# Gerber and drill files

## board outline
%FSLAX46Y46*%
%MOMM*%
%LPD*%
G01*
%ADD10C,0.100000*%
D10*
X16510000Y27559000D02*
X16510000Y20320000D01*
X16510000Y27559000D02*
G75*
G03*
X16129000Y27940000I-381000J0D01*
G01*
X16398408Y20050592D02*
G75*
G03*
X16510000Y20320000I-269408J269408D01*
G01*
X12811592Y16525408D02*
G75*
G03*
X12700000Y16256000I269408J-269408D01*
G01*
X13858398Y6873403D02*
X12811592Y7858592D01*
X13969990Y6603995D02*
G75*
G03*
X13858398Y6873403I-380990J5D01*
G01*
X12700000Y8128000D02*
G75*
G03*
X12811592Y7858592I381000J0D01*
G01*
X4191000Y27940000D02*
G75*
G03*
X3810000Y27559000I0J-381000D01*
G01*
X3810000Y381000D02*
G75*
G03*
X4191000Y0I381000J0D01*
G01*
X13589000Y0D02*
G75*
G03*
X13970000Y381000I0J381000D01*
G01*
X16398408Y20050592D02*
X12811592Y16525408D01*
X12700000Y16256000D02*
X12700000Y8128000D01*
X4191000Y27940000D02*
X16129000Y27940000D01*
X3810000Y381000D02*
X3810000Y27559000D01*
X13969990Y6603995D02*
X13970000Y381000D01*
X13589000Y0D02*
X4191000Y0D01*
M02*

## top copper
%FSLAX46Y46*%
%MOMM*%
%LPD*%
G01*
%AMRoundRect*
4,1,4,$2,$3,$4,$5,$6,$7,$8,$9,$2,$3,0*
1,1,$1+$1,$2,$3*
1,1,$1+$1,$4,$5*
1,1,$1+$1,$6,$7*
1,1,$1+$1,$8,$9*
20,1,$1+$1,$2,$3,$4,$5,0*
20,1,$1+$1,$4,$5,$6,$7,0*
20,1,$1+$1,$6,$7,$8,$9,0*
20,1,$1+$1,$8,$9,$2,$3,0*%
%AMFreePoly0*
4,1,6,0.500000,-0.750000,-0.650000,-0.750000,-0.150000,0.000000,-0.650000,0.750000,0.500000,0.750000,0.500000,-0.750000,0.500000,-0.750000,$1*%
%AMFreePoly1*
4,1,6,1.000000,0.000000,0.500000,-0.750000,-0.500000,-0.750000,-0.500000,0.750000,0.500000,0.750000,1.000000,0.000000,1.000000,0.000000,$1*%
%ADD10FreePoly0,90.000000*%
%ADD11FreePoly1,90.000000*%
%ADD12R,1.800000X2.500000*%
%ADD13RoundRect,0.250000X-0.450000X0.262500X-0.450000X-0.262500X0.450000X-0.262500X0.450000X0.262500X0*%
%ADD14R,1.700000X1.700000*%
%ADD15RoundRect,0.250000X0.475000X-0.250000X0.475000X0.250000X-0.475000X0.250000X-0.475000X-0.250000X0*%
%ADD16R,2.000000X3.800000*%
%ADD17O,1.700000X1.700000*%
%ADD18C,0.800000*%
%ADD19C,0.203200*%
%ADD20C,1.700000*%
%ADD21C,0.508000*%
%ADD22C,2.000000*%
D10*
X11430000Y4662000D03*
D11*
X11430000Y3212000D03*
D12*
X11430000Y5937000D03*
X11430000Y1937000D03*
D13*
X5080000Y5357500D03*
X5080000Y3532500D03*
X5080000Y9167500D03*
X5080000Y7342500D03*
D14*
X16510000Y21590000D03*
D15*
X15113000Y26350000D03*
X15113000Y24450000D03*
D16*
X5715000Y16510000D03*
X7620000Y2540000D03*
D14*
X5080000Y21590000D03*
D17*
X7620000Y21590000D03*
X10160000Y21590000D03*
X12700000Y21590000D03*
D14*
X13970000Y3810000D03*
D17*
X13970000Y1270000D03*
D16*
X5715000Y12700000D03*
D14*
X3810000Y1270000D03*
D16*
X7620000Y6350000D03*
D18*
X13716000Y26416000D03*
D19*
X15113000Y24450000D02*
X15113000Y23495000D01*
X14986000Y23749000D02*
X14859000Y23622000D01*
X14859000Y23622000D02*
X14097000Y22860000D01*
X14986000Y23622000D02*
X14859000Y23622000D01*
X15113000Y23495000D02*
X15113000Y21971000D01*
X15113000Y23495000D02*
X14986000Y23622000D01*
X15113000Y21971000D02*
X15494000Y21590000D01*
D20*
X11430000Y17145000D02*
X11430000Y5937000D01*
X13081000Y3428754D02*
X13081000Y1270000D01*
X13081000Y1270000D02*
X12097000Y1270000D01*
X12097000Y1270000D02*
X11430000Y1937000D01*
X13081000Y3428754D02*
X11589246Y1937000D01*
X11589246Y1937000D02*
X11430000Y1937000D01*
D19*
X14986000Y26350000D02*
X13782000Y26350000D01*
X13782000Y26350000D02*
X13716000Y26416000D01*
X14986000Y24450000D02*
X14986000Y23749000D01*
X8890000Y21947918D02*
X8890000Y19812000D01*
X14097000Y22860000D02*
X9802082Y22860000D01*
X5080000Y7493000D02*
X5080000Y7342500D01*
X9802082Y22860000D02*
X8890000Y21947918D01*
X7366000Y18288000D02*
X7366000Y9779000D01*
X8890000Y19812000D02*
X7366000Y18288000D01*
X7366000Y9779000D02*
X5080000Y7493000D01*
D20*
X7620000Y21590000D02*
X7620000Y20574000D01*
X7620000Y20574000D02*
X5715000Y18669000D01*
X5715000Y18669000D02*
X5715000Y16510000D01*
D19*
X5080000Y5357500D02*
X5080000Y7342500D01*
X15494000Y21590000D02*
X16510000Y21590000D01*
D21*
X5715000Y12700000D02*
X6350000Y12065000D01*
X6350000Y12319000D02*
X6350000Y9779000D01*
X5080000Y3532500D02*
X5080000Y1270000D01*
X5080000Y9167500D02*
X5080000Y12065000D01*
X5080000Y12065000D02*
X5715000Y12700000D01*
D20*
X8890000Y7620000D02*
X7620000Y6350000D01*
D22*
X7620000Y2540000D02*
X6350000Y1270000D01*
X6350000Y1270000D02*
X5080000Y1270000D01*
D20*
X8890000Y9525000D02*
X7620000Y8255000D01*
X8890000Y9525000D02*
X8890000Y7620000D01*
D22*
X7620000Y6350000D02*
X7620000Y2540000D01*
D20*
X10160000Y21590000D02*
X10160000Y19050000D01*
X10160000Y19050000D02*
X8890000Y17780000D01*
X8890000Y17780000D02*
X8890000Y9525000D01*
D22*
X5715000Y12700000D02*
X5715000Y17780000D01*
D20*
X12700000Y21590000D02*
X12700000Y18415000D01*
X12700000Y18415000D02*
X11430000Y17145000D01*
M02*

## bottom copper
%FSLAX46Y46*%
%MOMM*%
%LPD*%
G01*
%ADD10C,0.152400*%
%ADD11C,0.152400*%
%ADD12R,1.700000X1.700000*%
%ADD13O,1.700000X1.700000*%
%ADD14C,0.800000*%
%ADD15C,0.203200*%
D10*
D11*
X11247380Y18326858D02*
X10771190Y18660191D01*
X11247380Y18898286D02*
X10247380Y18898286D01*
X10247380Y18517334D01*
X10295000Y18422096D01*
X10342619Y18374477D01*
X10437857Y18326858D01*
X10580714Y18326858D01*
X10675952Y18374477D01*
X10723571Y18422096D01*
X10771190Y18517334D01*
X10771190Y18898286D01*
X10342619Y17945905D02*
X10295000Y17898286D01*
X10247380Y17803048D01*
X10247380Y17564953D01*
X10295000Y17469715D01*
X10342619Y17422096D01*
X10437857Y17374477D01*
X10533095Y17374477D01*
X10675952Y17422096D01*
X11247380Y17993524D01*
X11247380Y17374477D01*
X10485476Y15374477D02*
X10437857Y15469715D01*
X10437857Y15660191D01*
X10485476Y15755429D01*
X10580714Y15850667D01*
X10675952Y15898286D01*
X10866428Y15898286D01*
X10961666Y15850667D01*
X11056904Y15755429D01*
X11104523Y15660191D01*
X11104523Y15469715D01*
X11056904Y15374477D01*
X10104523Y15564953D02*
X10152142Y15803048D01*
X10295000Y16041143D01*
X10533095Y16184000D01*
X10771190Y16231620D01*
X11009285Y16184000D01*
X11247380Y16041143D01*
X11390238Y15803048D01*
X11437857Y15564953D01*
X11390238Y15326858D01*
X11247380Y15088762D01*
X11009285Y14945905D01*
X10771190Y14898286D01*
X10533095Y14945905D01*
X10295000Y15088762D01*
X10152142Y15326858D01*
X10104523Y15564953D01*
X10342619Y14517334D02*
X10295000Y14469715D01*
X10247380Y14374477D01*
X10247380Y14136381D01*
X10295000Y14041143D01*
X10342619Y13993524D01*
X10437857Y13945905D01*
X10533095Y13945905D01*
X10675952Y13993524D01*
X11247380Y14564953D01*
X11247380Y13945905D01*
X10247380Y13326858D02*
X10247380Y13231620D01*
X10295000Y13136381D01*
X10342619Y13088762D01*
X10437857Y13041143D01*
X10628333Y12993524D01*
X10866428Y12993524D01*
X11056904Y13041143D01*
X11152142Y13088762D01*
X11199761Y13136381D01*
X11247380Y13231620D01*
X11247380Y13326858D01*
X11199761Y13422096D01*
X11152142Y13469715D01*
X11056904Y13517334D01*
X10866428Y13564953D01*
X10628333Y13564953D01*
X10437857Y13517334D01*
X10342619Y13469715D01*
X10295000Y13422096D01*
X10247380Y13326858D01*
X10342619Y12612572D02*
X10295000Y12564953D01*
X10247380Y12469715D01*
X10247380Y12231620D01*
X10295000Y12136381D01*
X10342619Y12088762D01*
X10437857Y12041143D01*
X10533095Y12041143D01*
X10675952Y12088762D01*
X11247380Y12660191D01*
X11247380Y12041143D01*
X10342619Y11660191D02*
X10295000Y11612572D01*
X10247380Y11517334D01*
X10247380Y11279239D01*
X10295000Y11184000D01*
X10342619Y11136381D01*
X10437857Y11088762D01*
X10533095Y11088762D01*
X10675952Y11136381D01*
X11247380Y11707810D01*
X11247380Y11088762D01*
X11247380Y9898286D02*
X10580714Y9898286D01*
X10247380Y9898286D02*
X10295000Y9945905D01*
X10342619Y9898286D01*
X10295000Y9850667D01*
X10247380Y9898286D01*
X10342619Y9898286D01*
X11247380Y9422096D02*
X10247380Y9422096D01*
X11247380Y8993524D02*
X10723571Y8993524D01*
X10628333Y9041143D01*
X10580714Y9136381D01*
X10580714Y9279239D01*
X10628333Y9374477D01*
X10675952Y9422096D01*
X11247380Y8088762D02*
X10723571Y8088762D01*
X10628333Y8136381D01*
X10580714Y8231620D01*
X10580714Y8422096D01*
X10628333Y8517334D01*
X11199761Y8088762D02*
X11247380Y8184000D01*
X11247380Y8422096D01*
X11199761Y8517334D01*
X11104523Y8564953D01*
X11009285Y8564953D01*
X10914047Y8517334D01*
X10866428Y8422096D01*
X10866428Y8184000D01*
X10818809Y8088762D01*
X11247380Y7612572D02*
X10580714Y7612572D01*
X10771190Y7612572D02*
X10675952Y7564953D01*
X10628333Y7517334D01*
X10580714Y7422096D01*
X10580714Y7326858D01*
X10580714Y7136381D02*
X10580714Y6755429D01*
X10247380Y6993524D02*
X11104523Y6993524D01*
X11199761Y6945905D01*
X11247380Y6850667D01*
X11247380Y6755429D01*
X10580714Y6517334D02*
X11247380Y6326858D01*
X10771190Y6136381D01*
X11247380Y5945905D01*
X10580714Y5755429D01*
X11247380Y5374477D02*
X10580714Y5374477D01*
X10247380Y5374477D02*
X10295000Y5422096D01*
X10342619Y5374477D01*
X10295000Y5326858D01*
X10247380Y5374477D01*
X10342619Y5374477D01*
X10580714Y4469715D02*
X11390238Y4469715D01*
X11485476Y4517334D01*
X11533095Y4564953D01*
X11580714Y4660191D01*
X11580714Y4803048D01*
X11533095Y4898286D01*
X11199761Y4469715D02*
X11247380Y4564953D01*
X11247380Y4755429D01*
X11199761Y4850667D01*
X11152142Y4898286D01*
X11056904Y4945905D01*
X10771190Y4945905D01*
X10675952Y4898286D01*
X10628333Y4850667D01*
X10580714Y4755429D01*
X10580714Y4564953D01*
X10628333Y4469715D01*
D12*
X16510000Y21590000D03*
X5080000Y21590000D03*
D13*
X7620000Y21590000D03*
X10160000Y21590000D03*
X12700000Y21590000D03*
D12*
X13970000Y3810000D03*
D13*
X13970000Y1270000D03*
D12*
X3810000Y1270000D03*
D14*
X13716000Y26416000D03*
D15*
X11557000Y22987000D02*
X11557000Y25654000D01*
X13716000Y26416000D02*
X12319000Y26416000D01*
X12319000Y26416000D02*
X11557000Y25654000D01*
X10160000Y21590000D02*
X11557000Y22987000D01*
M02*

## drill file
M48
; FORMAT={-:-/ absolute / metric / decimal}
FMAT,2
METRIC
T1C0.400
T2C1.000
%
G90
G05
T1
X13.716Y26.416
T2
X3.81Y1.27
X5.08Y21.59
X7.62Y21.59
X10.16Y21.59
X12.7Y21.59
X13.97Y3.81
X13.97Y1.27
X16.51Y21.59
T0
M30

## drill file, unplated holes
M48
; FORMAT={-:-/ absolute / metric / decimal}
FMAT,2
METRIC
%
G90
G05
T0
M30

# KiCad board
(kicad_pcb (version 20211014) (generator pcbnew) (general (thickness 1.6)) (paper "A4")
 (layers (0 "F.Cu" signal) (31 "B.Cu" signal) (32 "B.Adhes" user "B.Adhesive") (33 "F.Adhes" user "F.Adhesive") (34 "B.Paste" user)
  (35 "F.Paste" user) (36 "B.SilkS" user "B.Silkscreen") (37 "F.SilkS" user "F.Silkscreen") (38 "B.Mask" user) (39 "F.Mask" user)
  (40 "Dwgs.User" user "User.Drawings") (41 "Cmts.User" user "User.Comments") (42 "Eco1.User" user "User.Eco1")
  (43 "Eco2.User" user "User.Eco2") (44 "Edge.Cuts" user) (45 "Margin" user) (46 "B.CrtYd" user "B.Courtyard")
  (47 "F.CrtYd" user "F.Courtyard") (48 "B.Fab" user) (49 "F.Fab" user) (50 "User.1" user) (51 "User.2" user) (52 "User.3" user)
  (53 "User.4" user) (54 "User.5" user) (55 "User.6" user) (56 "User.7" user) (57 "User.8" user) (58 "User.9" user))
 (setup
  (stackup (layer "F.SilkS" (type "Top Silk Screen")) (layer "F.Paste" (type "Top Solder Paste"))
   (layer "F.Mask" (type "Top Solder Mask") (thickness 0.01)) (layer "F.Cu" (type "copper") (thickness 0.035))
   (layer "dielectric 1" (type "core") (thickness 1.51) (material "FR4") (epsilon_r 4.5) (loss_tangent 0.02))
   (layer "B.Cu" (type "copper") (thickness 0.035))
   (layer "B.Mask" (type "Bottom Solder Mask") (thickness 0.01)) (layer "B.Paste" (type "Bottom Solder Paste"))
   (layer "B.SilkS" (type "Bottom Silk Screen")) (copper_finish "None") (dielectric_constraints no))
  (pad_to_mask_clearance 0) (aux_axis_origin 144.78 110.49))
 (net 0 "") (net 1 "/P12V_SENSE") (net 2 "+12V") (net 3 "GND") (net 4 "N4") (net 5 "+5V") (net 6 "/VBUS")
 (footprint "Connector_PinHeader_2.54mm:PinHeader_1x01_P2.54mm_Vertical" (layer "F.Cu") (at 161.29 88.9 90)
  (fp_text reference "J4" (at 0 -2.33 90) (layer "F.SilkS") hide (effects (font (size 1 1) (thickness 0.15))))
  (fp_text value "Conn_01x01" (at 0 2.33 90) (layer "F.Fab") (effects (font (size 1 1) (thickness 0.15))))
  (pad "1" thru_hole rect (at 0 0 90) (size 1.7 1.7) (drill 1) (layers *.Cu *.Mask) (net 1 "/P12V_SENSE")))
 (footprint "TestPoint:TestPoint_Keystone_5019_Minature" (layer "F.Cu") (at 150.495 93.98 90)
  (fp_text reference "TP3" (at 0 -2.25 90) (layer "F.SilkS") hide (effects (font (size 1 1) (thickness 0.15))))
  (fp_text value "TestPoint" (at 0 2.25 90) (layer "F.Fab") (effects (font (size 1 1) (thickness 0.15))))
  (pad "1" smd rect (at 0 0 90) (size 3.8 2) (layers "F.Cu" "F.Paste" "F.Mask") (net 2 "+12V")))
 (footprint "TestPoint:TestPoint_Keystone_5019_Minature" (layer "F.Cu") (at 152.4 107.95 90)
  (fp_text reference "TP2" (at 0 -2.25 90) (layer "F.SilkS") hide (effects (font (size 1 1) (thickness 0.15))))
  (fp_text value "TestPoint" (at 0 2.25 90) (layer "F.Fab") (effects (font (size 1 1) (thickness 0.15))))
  (pad "1" smd rect (at 0 0 90) (size 3.8 2) (layers "F.Cu" "F.Paste" "F.Mask") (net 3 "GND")))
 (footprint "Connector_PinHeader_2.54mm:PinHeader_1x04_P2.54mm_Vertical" (layer "F.Cu") (at 149.86 88.9 90)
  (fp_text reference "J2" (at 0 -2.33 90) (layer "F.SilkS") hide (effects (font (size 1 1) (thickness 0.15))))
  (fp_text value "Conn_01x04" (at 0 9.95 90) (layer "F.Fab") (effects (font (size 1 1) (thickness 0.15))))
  (pad "1" thru_hole rect (at 0 0 90) (size 1.7 1.7) (drill 1) (layers *.Cu *.Mask) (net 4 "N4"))
  (pad "2" thru_hole oval (at 0 2.54 90) (size 1.7 1.7) (drill 1) (layers *.Cu *.Mask) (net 2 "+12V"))
  (pad "3" thru_hole oval (at 0 5.08 90) (size 1.7 1.7) (drill 1) (layers *.Cu *.Mask) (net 3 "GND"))
  (pad "4" thru_hole oval (at 0 7.62 90) (size 1.7 1.7) (drill 1) (layers *.Cu *.Mask) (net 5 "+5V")))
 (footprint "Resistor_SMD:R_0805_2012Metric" (layer "F.Cu") (at 149.86 102.235 -90)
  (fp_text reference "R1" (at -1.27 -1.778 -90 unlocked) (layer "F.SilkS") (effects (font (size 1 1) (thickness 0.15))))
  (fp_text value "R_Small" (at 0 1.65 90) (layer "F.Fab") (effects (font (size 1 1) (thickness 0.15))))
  (pad "1" smd roundrect (at -0.9125 0 270) (size 1.025 1.4) (layers "F.Cu" "F.Paste" "F.Mask") (roundrect_rratio 0.243902439)
   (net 2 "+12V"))
  (pad "2" smd roundrect (at 0.9125 0 270) (size 1.025 1.4) (layers "F.Cu" "F.Paste" "F.Mask") (roundrect_rratio 0.243902439)
   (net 1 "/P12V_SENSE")))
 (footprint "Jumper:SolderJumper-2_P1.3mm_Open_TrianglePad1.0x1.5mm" (layer "F.Cu") (at 156.21 106.553 90)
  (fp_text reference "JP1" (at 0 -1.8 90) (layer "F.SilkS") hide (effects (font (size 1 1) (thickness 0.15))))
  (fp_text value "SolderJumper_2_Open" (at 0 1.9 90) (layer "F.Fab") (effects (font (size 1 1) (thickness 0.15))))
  (pad "1" smd custom (at -0.725 0 90) (size 0.3 0.3) (layers "F.Cu" "F.Mask") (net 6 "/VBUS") (zone_connect 2)
   (options (clearance outline) (anchor rect)) (primitives))
  (pad "2" smd custom (at 0.725 0 90) (size 0.3 0.3) (layers "F.Cu" "F.Mask") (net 5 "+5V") (zone_connect 2)
   (options (clearance outline) (anchor rect)) (primitives)))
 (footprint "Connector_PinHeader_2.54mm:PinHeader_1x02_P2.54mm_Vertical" (layer "F.Cu") (at 158.75 106.68)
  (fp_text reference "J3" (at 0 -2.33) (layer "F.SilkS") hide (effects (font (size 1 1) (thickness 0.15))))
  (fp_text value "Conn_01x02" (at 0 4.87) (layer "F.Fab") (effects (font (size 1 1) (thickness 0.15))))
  (pad "1" thru_hole rect (at 0 0) (size 1.7 1.7) (drill 1) (layers *.Cu *.Mask) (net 6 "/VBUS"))
  (pad "2" thru_hole oval (at 0 2.54) (size 1.7 1.7) (drill 1) (layers *.Cu *.Mask) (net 6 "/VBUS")))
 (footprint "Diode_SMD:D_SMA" (layer "F.Cu") (at 156.21 106.553 90)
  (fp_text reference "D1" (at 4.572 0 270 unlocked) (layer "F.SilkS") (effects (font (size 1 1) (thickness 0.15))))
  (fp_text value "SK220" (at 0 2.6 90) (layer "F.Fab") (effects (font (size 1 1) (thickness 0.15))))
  (pad "1" smd rect (at -2 0 90) (size 2.5 1.8) (layers "F.Cu" "F.Paste" "F.Mask") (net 6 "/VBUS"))
  (pad "2" smd rect (at 2 0 90) (size 2.5 1.8) (layers "F.Cu" "F.Paste" "F.Mask") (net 5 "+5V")))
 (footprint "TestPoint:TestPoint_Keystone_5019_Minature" (layer "F.Cu") (at 150.495 97.79 90)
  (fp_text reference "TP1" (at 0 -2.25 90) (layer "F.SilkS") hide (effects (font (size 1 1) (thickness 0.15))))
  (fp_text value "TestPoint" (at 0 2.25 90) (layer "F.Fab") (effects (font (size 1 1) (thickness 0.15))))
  (pad "1" smd rect (at 0 0 90) (size 3.8 2) (layers "F.Cu" "F.Paste" "F.Mask") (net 2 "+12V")))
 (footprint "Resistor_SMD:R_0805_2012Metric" (layer "F.Cu") (at 149.86 106.045 -90)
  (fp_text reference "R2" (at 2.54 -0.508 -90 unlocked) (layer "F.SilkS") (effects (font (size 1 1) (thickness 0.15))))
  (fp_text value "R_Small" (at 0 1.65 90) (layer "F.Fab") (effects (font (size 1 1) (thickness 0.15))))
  (pad "1" smd roundrect (at -0.9125 0 270) (size 1.025 1.4) (layers "F.Cu" "F.Paste" "F.Mask") (roundrect_rratio 0.243902439)
   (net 1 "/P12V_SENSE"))
  (pad "2" smd roundrect (at 0.9125 0 270) (size 1.025 1.4) (layers "F.Cu" "F.Paste" "F.Mask") (roundrect_rratio 0.243902439) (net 3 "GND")))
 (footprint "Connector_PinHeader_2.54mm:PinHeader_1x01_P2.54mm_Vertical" (layer "F.Cu") (at 148.59 109.22)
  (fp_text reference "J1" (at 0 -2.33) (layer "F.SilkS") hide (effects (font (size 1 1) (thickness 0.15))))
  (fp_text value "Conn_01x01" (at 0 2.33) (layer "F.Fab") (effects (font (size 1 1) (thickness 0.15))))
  (pad "1" thru_hole rect (at 0 0) (size 1.7 1.7) (drill 1) (layers *.Cu *.Mask) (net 3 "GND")))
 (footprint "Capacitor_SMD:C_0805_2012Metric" (layer "F.Cu") (at 159.893 85.09 90)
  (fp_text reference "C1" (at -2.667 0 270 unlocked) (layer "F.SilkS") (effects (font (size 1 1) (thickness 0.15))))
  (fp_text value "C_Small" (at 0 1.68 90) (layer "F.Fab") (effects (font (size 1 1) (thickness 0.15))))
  (pad "1" smd roundrect (at -0.95 0 90) (size 1 1.45) (layers "F.Cu" "F.Paste" "F.Mask") (roundrect_rratio 0.25) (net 1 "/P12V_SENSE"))
  (pad "2" smd roundrect (at 0.95 0 90) (size 1 1.45) (layers "F.Cu" "F.Paste" "F.Mask") (roundrect_rratio 0.25) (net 3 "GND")))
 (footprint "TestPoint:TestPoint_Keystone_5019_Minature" (layer "F.Cu") (at 152.4 104.14 90)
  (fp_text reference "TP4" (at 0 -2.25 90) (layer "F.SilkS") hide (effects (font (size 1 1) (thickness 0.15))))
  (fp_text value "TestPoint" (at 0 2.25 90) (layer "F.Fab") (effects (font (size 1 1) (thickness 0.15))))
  (pad "1" smd rect (at 0 0 90) (size 3.8 2) (layers "F.Cu" "F.Paste" "F.Mask") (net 3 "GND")))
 (gr_line (start 161.29 82.931) (end 161.29 90.17) (layer "Edge.Cuts") (width 0.1))
 (gr_line (start 158.638398 103.616597) (end 157.591592 102.631408) (layer "Edge.Cuts") (width 0.1))
 (gr_line (start 161.178408 90.439408) (end 157.591592 93.964592) (layer "Edge.Cuts") (width 0.1))
 (gr_arc (start 158.75 110.109) (mid 158.638408 110.378408) (end 158.369 110.49) (layer "Edge.Cuts") (width 0.1))
 (gr_arc (start 148.971 110.49) (mid 148.701592 110.378408) (end 148.59 110.109) (layer "Edge.Cuts") (width 0.1))
 (gr_line (start 157.48 94.234) (end 157.48 102.362) (layer "Edge.Cuts") (width 0.1))
 (gr_arc (start 158.638398 103.616597) (mid 158.720989 103.740202) (end 158.74999 103.886005) (layer "Edge.Cuts") (width 0.1))
 (gr_line (start 148.971 82.55) (end 160.909 82.55) (layer "Edge.Cuts") (width 0.1))
 (gr_arc (start 157.591592 102.631408) (mid 157.509001 102.507803) (end 157.48 102.362) (layer "Edge.Cuts") (width 0.1))
 (gr_arc (start 157.48 94.234) (mid 157.509002 94.088198) (end 157.591592 93.964592) (layer "Edge.Cuts") (width 0.1))
 (gr_line (start 148.59 110.109) (end 148.59 82.931) (layer "Edge.Cuts") (width 0.1))
 (gr_arc (start 148.59 82.931) (mid 148.701592 82.661592) (end 148.971 82.55) (layer "Edge.Cuts") (width 0.1))
 (gr_line (start 158.74999 103.886005) (end 158.75 110.109) (layer "Edge.Cuts") (width 0.1))
 (gr_line (start 158.369 110.49) (end 148.971 110.49) (layer "Edge.Cuts") (width 0.1))
 (gr_arc (start 161.29 90.17) (mid 161.260998 90.315802) (end 161.178408 90.439408) (layer "Edge.Cuts") (width 0.1))
 (gr_arc (start 160.909 82.55) (mid 161.178408 82.661592) (end 161.29 82.931) (layer "Edge.Cuts") (width 0.1))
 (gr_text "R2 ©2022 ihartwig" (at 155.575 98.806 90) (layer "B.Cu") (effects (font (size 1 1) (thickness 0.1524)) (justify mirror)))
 (segment (start 153.67 102.87) (end 152.4 104.14) (width 1.7) (layer "F.Cu") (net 3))
 (segment (start 152.4 107.95) (end 151.13 109.22) (width 2) (layer "F.Cu") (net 3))
 (segment (start 151.13 109.22) (end 149.86 109.22) (width 2) (layer "F.Cu") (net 3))
 (segment (start 153.67 100.965) (end 152.4 102.235) (width 1.7) (layer "F.Cu") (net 3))
 (segment (start 153.67 100.965) (end 153.67 102.87) (width 1.7) (layer "F.Cu") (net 3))
 (segment (start 159.766 84.14) (end 158.562 84.14) (width 0.2032) (layer "F.Cu") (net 3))
 (segment (start 152.4 104.14) (end 152.4 107.95) (width 2) (layer "F.Cu") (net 3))
 (segment (start 154.94 88.9) (end 154.94 91.44) (width 1.7) (layer "F.Cu") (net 3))
 (segment (start 149.86 106.9575) (end 149.86 109.22) (width 0.508) (layer "F.Cu") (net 3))
 (segment (start 154.94 91.44) (end 153.67 92.71) (width 1.7) (layer "F.Cu") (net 3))
 (segment (start 153.67 92.71) (end 153.67 100.965) (width 1.7) (layer "F.Cu") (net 3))
 (segment (start 158.562 84.14) (end 158.496 84.074) (width 0.2032) (layer "F.Cu") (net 3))
 (via (at 158.496 84.074) (size 0.8) (drill 0.4) (layers "F.Cu" "B.Cu") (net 3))
 (segment (start 156.337 87.503) (end 156.337 84.836) (width 0.2032) (layer "B.Cu") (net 3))
 (segment (start 158.496 84.074) (end 157.099 84.074) (width 0.2032) (layer "B.Cu") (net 3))
 (segment (start 157.099 84.074) (end 156.337 84.836) (width 0.2032) (layer "B.Cu") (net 3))
 (segment (start 154.94 88.9) (end 156.337 87.503) (width 0.2032) (layer "B.Cu") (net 3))
 (segment (start 150.495 91.821) (end 150.495 93.98) (width 1.7) (layer "F.Cu") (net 2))
 (segment (start 152.4 89.916) (end 150.495 91.821) (width 1.7) (layer "F.Cu") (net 2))
 (segment (start 150.495 97.79) (end 151.13 98.425) (width 0.508) (layer "F.Cu") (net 2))
 (segment (start 151.13 98.171) (end 151.13 100.711) (width 0.508) (layer "F.Cu") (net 2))
 (segment (start 149.86 98.425) (end 150.495 97.79) (width 0.508) (layer "F.Cu") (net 2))
 (segment (start 149.86 101.3225) (end 149.86 98.425) (width 0.508) (layer "F.Cu") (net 2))
 (segment (start 152.4 88.9) (end 152.4 89.916) (width 1.7) (layer "F.Cu") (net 2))
 (segment (start 150.495 97.79) (end 150.495 92.71) (width 2) (layer "F.Cu") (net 2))
 (segment (start 157.48 88.9) (end 157.48 92.075) (width 1.7) (layer "F.Cu") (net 5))
 (segment (start 156.21 93.345) (end 156.21 104.553) (width 1.7) (layer "F.Cu") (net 5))
 (segment (start 157.48 92.075) (end 156.21 93.345) (width 1.7) (layer "F.Cu") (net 5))
 (segment (start 154.582082 87.63) (end 153.67 88.542082) (width 0.2032) (layer "F.Cu") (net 1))
 (segment (start 159.893 88.519) (end 160.274 88.9) (width 0.2032) (layer "F.Cu") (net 1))
 (segment (start 153.67 88.542082) (end 153.67 90.678) (width 0.2032) (layer "F.Cu") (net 1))
 (segment (start 159.893 86.04) (end 159.893 86.995) (width 0.2032) (layer "F.Cu") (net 1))
 (segment (start 149.86 105.1325) (end 149.86 103.1475) (width 0.2032) (layer "F.Cu") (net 1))
 (segment (start 152.146 92.202) (end 152.146 100.711) (width 0.2032) (layer "F.Cu") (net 1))
 (segment (start 153.67 90.678) (end 152.146 92.202) (width 0.2032) (layer "F.Cu") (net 1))
 (segment (start 159.766 86.04) (end 159.766 86.741) (width 0.2032) (layer "F.Cu") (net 1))
 (segment (start 159.893 86.995) (end 159.893 88.519) (width 0.2032) (layer "F.Cu") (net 1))
 (segment (start 158.877 87.63) (end 154.582082 87.63) (width 0.2032) (layer "F.Cu") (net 1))
 (segment (start 159.766 86.741) (end 159.639 86.868) (width 0.2032) (layer "F.Cu") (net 1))
 (segment (start 152.146 100.711) (end 149.86 102.997) (width 0.2032) (layer "F.Cu") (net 1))
 (segment (start 160.274 88.9) (end 161.29 88.9) (width 0.2032) (layer "F.Cu") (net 1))
 (segment (start 159.766 86.868) (end 159.639 86.868) (width 0.2032) (layer "F.Cu") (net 1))
 (segment (start 159.639 86.868) (end 158.877 87.63) (width 0.2032) (layer "F.Cu") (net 1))
 (segment (start 149.86 102.997) (end 149.86 103.1475) (width 0.2032) (layer "F.Cu") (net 1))
 (segment (start 159.893 86.995) (end 159.766 86.868) (width 0.2032) (layer "F.Cu") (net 1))
 (segment (start 156.369246 108.553) (end 156.21 108.553) (width 1.7) (layer "F.Cu") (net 6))
 (segment (start 157.861 107.061246) (end 157.861 109.22) (width 1.7) (layer "F.Cu") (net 6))
 (segment (start 157.861 109.22) (end 156.877 109.22) (width 1.7) (layer "F.Cu") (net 6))
 (segment (start 156.877 109.22) (end 156.21 108.553) (width 1.7) (layer "F.Cu") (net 6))
 (segment (start 157.861 107.061246) (end 156.369246 108.553) (width 1.7) (layer "F.Cu") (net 6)))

